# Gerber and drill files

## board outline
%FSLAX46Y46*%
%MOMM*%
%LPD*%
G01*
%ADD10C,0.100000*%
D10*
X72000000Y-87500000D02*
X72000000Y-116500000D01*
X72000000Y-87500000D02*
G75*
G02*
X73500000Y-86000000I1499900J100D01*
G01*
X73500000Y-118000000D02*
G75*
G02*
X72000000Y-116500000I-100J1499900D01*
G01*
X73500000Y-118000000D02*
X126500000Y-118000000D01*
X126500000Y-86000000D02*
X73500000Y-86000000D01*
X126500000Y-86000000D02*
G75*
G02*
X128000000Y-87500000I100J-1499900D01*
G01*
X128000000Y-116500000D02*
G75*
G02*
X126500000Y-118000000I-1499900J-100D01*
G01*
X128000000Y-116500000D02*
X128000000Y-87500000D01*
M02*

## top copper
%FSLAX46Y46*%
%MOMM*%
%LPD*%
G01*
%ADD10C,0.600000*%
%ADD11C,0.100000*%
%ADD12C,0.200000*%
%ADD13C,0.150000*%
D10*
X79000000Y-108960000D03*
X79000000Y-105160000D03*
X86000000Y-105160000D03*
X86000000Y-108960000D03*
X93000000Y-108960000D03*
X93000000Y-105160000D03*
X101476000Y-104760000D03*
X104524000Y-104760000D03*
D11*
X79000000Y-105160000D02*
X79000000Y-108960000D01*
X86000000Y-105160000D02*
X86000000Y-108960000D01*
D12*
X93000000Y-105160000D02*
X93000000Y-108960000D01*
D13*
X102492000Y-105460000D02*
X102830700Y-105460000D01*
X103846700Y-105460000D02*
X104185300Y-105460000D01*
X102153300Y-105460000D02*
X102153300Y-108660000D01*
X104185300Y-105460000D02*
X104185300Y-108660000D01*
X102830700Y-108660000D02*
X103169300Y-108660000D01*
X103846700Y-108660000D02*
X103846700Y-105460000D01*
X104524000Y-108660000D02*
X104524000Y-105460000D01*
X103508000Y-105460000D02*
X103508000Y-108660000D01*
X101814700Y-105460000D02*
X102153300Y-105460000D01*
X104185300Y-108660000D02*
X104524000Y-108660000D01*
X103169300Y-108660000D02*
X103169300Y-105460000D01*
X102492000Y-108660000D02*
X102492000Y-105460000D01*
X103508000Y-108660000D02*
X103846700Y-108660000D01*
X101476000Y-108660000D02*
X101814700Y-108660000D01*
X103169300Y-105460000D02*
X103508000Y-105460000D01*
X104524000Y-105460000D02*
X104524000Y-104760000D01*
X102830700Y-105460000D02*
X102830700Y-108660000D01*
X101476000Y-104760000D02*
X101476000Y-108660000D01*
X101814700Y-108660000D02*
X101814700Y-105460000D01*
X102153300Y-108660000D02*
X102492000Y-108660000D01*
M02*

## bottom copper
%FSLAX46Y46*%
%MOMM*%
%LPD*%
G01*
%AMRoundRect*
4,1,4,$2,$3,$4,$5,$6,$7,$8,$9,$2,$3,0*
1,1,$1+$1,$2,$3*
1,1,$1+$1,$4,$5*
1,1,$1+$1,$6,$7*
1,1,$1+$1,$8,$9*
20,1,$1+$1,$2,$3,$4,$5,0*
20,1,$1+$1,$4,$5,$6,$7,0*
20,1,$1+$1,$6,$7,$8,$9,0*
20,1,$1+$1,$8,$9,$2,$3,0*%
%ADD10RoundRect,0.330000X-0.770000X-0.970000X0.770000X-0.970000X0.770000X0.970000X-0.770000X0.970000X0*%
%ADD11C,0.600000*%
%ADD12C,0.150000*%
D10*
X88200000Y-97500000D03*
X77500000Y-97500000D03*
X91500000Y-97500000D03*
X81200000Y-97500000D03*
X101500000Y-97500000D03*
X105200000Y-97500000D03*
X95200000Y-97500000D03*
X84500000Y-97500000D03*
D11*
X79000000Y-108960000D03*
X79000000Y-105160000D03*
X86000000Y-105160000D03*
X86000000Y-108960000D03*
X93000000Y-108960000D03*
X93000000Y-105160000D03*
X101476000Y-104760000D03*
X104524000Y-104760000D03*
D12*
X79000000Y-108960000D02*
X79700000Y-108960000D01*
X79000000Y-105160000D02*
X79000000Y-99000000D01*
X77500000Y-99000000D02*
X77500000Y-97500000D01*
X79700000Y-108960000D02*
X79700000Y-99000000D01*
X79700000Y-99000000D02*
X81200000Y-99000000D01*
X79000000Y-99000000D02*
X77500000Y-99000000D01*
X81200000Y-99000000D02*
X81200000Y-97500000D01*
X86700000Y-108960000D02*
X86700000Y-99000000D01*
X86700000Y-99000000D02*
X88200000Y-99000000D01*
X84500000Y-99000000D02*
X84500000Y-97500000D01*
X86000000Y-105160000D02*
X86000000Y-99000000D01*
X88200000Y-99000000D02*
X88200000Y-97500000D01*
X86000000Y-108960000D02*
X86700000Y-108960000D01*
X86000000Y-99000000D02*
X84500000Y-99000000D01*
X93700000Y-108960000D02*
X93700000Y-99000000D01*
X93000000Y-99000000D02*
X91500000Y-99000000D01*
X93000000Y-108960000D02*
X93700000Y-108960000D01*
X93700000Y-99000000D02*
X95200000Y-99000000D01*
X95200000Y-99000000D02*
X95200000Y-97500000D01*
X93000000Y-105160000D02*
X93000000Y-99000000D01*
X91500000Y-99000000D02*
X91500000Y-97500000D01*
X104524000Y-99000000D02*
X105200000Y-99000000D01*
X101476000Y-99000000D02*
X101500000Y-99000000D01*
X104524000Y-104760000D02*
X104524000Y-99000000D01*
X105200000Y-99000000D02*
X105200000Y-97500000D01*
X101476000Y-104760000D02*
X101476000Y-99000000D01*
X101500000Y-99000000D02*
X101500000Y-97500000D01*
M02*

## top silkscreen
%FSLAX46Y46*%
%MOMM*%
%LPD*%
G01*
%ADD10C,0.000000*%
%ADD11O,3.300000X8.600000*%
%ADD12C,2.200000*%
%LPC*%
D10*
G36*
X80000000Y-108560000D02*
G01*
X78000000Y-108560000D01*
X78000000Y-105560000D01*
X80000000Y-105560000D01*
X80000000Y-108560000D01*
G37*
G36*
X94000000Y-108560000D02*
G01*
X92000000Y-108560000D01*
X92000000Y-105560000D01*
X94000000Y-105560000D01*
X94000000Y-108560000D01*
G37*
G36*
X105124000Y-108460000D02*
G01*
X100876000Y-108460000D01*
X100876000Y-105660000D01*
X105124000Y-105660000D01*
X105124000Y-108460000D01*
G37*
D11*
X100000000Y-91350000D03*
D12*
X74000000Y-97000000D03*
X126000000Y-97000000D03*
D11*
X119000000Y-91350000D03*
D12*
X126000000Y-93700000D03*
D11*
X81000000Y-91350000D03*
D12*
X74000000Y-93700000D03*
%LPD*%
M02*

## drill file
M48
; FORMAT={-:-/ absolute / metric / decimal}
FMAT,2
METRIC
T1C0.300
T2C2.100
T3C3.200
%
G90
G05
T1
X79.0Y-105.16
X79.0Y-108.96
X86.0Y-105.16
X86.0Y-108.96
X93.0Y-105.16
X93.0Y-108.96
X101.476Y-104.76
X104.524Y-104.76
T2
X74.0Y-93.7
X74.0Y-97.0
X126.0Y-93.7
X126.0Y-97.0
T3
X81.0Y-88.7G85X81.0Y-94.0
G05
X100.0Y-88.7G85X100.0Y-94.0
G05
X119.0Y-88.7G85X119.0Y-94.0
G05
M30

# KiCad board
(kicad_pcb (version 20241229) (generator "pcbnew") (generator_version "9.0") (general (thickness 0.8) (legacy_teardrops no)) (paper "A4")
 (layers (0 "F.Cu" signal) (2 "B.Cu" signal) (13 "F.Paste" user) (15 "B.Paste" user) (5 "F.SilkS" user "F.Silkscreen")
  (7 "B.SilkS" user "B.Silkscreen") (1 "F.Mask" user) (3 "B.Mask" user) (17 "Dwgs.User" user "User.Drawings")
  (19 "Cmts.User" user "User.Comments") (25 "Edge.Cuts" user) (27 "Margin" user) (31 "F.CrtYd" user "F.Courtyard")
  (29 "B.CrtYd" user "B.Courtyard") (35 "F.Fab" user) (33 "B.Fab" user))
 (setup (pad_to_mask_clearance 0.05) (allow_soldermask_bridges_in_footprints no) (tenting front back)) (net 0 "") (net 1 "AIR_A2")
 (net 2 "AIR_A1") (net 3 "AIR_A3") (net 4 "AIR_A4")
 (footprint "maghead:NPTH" (layer "F.Cu") (at 100 91.35)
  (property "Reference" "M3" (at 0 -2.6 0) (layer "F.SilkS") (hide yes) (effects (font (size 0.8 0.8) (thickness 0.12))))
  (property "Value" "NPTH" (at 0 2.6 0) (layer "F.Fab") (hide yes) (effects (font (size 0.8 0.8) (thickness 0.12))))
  (pad "" np_thru_hole oval (at 0 0) (size 3.2 8.5) (drill oval 3.2 8.5) (layers "*.Cu" "*.Mask")))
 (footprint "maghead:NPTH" (layer "F.Cu") (at 74 97)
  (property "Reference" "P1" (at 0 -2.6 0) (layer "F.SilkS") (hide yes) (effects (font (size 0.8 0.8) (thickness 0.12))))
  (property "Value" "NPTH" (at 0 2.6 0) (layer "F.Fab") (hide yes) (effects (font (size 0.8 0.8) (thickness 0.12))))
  (pad "" np_thru_hole circle (at 0 0) (size 2.1 2.1) (drill 2.1) (layers "*.Cu" "*.Mask")))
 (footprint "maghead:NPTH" (layer "F.Cu") (at 126 97)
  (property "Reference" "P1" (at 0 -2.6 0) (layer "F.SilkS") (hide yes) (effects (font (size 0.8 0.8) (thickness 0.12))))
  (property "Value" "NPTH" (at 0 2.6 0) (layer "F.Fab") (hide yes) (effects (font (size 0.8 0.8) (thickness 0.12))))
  (pad "" np_thru_hole circle (at 0 0) (size 2.1 2.1) (drill 2.1) (layers "*.Cu" "*.Mask")))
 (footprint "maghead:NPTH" (layer "F.Cu") (at 119 91.35)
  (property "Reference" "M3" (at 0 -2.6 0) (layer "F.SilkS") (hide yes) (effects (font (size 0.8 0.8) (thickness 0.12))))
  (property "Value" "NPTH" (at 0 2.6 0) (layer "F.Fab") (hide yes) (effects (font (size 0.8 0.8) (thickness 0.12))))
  (pad "" np_thru_hole oval (at 0 0) (size 3.2 8.5) (drill oval 3.2 8.5) (layers "*.Cu" "*.Mask")))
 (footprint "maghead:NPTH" (layer "F.Cu") (at 126 93.7)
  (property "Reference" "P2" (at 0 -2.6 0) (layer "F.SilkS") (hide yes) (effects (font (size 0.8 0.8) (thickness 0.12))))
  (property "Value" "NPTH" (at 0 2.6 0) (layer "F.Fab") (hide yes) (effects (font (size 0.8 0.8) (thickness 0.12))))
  (pad "" np_thru_hole circle (at 0 0) (size 2.1 2.1) (drill 2.1) (layers "*.Cu" "*.Mask")))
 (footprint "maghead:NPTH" (layer "F.Cu") (at 81 91.35)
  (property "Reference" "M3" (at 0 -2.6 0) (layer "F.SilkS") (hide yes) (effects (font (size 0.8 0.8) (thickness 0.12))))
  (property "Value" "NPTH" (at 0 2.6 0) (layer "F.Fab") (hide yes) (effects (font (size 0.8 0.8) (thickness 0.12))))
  (pad "" np_thru_hole oval (at 0 0) (size 3.2 8.5) (drill oval 3.2 8.5) (layers "*.Cu" "*.Mask")))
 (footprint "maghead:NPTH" (layer "F.Cu") (at 74 93.7)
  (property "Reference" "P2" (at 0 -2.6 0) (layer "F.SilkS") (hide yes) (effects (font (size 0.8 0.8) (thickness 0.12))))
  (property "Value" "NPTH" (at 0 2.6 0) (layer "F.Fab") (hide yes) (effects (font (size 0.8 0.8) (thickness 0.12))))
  (pad "" np_thru_hole circle (at 0 0) (size 2.1 2.1) (drill 2.1) (layers "*.Cu" "*.Mask")))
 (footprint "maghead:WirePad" (layer "B.Cu") (at 88.2 97.5)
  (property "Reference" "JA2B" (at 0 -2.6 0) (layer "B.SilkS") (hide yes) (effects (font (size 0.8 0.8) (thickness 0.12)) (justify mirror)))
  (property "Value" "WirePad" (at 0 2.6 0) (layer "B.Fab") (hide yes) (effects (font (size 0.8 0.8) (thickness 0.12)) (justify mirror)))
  (pad "1" smd roundrect (at 0 0) (size 2.2 2.6) (layers "B.Cu" "B.Mask") (roundrect_rratio 0.15) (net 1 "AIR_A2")))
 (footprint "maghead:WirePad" (layer "B.Cu") (at 77.5 97.5)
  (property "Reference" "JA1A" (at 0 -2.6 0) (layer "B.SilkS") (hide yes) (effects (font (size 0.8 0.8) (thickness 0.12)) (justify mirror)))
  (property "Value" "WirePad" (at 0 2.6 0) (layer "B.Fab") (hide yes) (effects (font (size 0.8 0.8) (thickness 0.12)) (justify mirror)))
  (pad "1" smd roundrect (at 0 0) (size 2.2 2.6) (layers "B.Cu" "B.Mask") (roundrect_rratio 0.15) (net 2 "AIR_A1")))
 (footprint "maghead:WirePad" (layer "B.Cu") (at 91.5 97.5)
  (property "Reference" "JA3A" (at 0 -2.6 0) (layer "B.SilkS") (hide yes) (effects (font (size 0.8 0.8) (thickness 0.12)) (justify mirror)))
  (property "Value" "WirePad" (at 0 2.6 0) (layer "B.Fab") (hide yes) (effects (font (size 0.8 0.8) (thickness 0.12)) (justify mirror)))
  (pad "1" smd roundrect (at 0 0) (size 2.2 2.6) (layers "B.Cu" "B.Mask") (roundrect_rratio 0.15) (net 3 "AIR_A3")))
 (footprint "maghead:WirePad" (layer "B.Cu") (at 81.2 97.5)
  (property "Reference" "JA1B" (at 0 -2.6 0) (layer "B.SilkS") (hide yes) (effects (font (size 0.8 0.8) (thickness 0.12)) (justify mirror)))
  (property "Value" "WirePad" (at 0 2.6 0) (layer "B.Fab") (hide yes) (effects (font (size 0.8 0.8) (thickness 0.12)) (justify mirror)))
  (pad "1" smd roundrect (at 0 0) (size 2.2 2.6) (layers "B.Cu" "B.Mask") (roundrect_rratio 0.15) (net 2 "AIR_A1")))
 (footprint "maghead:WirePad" (layer "B.Cu") (at 101.5 97.5)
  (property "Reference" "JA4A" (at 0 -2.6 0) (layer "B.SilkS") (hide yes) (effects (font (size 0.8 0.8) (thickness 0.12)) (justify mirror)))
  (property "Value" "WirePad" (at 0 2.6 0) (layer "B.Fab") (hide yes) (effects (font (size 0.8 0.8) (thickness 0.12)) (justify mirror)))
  (pad "1" smd roundrect (at 0 0) (size 2.2 2.6) (layers "B.Cu" "B.Mask") (roundrect_rratio 0.15) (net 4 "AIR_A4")))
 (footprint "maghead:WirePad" (layer "B.Cu") (at 105.2 97.5)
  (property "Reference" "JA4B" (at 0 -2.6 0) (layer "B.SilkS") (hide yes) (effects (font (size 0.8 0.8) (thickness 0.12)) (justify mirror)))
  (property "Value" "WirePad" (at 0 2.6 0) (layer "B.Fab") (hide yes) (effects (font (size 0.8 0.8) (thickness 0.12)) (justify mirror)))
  (pad "1" smd roundrect (at 0 0) (size 2.2 2.6) (layers "B.Cu" "B.Mask") (roundrect_rratio 0.15) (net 4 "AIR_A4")))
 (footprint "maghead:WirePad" (layer "B.Cu") (at 95.2 97.5)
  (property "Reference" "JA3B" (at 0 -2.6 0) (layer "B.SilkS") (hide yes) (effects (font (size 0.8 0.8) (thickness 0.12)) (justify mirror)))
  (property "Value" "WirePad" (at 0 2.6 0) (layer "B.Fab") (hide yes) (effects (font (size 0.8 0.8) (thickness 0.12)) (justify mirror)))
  (pad "1" smd roundrect (at 0 0) (size 2.2 2.6) (layers "B.Cu" "B.Mask") (roundrect_rratio 0.15) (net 3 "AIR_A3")))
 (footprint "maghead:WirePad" (layer "B.Cu") (at 84.5 97.5)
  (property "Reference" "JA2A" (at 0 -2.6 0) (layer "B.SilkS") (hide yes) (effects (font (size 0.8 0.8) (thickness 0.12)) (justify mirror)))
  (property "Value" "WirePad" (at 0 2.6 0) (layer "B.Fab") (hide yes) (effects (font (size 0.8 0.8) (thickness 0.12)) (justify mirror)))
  (pad "1" smd roundrect (at 0 0) (size 2.2 2.6) (layers "B.Cu" "B.Mask") (roundrect_rratio 0.15) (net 1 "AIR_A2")))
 (gr_line (start 72 87.5) (end 72 116.5) (stroke (width 0.1) (type solid)) (layer "Edge.Cuts"))
 (gr_arc (start 72 87.5) (mid 72.439311 86.439311) (end 73.5 86) (stroke (width 0.1) (type solid)) (layer "Edge.Cuts"))
 (gr_arc (start 73.5 118) (mid 72.439311 117.560689) (end 72 116.5) (stroke (width 0.1) (type solid)) (layer "Edge.Cuts"))
 (gr_line (start 73.5 118) (end 126.5 118) (stroke (width 0.1) (type solid)) (layer "Edge.Cuts"))
 (gr_line (start 126.5 86) (end 73.5 86) (stroke (width 0.1) (type solid)) (layer "Edge.Cuts"))
 (gr_arc (start 126.5 86) (mid 127.560689 86.439311) (end 128 87.5) (stroke (width 0.1) (type solid)) (layer "Edge.Cuts"))
 (gr_arc (start 128 116.5) (mid 127.560689 117.560689) (end 126.5 118) (stroke (width 0.1) (type solid)) (layer "Edge.Cuts"))
 (gr_line (start 128 116.5) (end 128 87.5) (stroke (width 0.1) (type solid)) (layer "Edge.Cuts"))
 (segment (start 79 105.16) (end 79 108.96) (width 0.1) (layer "F.Cu") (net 2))
 (via (at 79 108.96) (size 0.6) (drill 0.3) (layers "F.Cu" "B.Cu") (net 2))
 (via (at 79 105.16) (size 0.6) (drill 0.3) (layers "F.Cu" "B.Cu") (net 2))
 (segment (start 79 108.96) (end 79.7 108.96) (width 0.15) (layer "B.Cu") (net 2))
 (segment (start 79 105.16) (end 79 99) (width 0.15) (layer "B.Cu") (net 2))
 (segment (start 77.5 99) (end 77.5 97.5) (width 0.15) (layer "B.Cu") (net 2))
 (segment (start 79.7 108.96) (end 79.7 99) (width 0.15) (layer "B.Cu") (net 2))
 (segment (start 79.7 99) (end 81.2 99) (width 0.15) (layer "B.Cu") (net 2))
 (segment (start 79 99) (end 77.5 99) (width 0.15) (layer "B.Cu") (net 2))
 (segment (start 81.2 99) (end 81.2 97.5) (width 0.15) (layer "B.Cu") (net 2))
 (segment (start 86 105.16) (end 86 108.96) (width 0.1) (layer "F.Cu") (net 1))
 (via (at 86 105.16) (size 0.6) (drill 0.3) (layers "F.Cu" "B.Cu") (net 1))
 (via (at 86 108.96) (size 0.6) (drill 0.3) (layers "F.Cu" "B.Cu") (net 1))
 (segment (start 86.7 108.96) (end 86.7 99) (width 0.15) (layer "B.Cu") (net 1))
 (segment (start 86.7 99) (end 88.2 99) (width 0.15) (layer "B.Cu") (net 1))
 (segment (start 84.5 99) (end 84.5 97.5) (width 0.15) (layer "B.Cu") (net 1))
 (segment (start 86 105.16) (end 86 99) (width 0.15) (layer "B.Cu") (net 1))
 (segment (start 88.2 99) (end 88.2 97.5) (width 0.15) (layer "B.Cu") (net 1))
 (segment (start 86 108.96) (end 86.7 108.96) (width 0.15) (layer "B.Cu") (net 1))
 (segment (start 86 99) (end 84.5 99) (width 0.15) (layer "B.Cu") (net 1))
 (segment (start 93 105.16) (end 93 108.96) (width 0.2) (layer "F.Cu") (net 3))
 (via (at 93 108.96) (size 0.6) (drill 0.3) (layers "F.Cu" "B.Cu") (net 3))
 (via (at 93 105.16) (size 0.6) (drill 0.3) (layers "F.Cu" "B.Cu") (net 3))
 (segment (start 93.7 108.96) (end 93.7 99) (width 0.15) (layer "B.Cu") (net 3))
 (segment (start 93 99) (end 91.5 99) (width 0.15) (layer "B.Cu") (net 3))
 (segment (start 93 108.96) (end 93.7 108.96) (width 0.15) (layer "B.Cu") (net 3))
 (segment (start 93.7 99) (end 95.2 99) (width 0.15) (layer "B.Cu") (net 3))
 (segment (start 95.2 99) (end 95.2 97.5) (width 0.15) (layer "B.Cu") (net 3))
 (segment (start 93 105.16) (end 93 99) (width 0.15) (layer "B.Cu") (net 3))
 (segment (start 91.5 99) (end 91.5 97.5) (width 0.15) (layer "B.Cu") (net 3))
 (segment (start 102.492 105.46) (end 102.8307 105.46) (width 0.15) (layer "F.Cu") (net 4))
 (segment (start 103.8467 105.46) (end 104.1853 105.46) (width 0.15) (layer "F.Cu") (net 4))
 (segment (start 102.1533 105.46) (end 102.1533 108.66) (width 0.15) (layer "F.Cu") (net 4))
 (segment (start 104.1853 105.46) (end 104.1853 108.66) (width 0.15) (layer "F.Cu") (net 4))
 (segment (start 102.8307 108.66) (end 103.1693 108.66) (width 0.15) (layer "F.Cu") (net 4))
 (segment (start 103.8467 108.66) (end 103.8467 105.46) (width 0.15) (layer "F.Cu") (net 4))
 (segment (start 104.524 108.66) (end 104.524 105.46) (width 0.15) (layer "F.Cu") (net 4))
 (segment (start 103.508 105.46) (end 103.508 108.66) (width 0.15) (layer "F.Cu") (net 4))
 (segment (start 101.8147 105.46) (end 102.1533 105.46) (width 0.15) (layer "F.Cu") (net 4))
 (segment (start 104.1853 108.66) (end 104.524 108.66) (width 0.15) (layer "F.Cu") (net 4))
 (segment (start 103.1693 108.66) (end 103.1693 105.46) (width 0.15) (layer "F.Cu") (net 4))
 (segment (start 102.492 108.66) (end 102.492 105.46) (width 0.15) (layer "F.Cu") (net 4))
 (segment (start 103.508 108.66) (end 103.8467 108.66) (width 0.15) (layer "F.Cu") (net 4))
 (segment (start 101.476 108.66) (end 101.8147 108.66) (width 0.15) (layer "F.Cu") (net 4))
 (segment (start 103.1693 105.46) (end 103.508 105.46) (width 0.15) (layer "F.Cu") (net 4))
 (segment (start 104.524 105.46) (end 104.524 104.76) (width 0.15) (layer "F.Cu") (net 4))
 (segment (start 102.8307 105.46) (end 102.8307 108.66) (width 0.15) (layer "F.Cu") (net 4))
 (segment (start 101.476 104.76) (end 101.476 108.66) (width 0.15) (layer "F.Cu") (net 4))
 (segment (start 101.8147 108.66) (end 101.8147 105.46) (width 0.15) (layer "F.Cu") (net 4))
 (segment (start 102.1533 108.66) (end 102.492 108.66) (width 0.15) (layer "F.Cu") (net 4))
 (via (at 101.476 104.76) (size 0.6) (drill 0.3) (layers "F.Cu" "B.Cu") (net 4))
 (via (at 104.524 104.76) (size 0.6) (drill 0.3) (layers "F.Cu" "B.Cu") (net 4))
 (segment (start 104.524 99) (end 105.2 99) (width 0.15) (layer "B.Cu") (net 4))
 (segment (start 101.476 99) (end 101.5 99) (width 0.15) (layer "B.Cu") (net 4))
 (segment (start 104.524 104.76) (end 104.524 99) (width 0.15) (layer "B.Cu") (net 4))
 (segment (start 105.2 99) (end 105.2 97.5) (width 0.15) (layer "B.Cu") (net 4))
 (segment (start 101.476 104.76) (end 101.476 99) (width 0.15) (layer "B.Cu") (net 4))
 (segment (start 101.5 99) (end 101.5 97.5) (width 0.15) (layer "B.Cu") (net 4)))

